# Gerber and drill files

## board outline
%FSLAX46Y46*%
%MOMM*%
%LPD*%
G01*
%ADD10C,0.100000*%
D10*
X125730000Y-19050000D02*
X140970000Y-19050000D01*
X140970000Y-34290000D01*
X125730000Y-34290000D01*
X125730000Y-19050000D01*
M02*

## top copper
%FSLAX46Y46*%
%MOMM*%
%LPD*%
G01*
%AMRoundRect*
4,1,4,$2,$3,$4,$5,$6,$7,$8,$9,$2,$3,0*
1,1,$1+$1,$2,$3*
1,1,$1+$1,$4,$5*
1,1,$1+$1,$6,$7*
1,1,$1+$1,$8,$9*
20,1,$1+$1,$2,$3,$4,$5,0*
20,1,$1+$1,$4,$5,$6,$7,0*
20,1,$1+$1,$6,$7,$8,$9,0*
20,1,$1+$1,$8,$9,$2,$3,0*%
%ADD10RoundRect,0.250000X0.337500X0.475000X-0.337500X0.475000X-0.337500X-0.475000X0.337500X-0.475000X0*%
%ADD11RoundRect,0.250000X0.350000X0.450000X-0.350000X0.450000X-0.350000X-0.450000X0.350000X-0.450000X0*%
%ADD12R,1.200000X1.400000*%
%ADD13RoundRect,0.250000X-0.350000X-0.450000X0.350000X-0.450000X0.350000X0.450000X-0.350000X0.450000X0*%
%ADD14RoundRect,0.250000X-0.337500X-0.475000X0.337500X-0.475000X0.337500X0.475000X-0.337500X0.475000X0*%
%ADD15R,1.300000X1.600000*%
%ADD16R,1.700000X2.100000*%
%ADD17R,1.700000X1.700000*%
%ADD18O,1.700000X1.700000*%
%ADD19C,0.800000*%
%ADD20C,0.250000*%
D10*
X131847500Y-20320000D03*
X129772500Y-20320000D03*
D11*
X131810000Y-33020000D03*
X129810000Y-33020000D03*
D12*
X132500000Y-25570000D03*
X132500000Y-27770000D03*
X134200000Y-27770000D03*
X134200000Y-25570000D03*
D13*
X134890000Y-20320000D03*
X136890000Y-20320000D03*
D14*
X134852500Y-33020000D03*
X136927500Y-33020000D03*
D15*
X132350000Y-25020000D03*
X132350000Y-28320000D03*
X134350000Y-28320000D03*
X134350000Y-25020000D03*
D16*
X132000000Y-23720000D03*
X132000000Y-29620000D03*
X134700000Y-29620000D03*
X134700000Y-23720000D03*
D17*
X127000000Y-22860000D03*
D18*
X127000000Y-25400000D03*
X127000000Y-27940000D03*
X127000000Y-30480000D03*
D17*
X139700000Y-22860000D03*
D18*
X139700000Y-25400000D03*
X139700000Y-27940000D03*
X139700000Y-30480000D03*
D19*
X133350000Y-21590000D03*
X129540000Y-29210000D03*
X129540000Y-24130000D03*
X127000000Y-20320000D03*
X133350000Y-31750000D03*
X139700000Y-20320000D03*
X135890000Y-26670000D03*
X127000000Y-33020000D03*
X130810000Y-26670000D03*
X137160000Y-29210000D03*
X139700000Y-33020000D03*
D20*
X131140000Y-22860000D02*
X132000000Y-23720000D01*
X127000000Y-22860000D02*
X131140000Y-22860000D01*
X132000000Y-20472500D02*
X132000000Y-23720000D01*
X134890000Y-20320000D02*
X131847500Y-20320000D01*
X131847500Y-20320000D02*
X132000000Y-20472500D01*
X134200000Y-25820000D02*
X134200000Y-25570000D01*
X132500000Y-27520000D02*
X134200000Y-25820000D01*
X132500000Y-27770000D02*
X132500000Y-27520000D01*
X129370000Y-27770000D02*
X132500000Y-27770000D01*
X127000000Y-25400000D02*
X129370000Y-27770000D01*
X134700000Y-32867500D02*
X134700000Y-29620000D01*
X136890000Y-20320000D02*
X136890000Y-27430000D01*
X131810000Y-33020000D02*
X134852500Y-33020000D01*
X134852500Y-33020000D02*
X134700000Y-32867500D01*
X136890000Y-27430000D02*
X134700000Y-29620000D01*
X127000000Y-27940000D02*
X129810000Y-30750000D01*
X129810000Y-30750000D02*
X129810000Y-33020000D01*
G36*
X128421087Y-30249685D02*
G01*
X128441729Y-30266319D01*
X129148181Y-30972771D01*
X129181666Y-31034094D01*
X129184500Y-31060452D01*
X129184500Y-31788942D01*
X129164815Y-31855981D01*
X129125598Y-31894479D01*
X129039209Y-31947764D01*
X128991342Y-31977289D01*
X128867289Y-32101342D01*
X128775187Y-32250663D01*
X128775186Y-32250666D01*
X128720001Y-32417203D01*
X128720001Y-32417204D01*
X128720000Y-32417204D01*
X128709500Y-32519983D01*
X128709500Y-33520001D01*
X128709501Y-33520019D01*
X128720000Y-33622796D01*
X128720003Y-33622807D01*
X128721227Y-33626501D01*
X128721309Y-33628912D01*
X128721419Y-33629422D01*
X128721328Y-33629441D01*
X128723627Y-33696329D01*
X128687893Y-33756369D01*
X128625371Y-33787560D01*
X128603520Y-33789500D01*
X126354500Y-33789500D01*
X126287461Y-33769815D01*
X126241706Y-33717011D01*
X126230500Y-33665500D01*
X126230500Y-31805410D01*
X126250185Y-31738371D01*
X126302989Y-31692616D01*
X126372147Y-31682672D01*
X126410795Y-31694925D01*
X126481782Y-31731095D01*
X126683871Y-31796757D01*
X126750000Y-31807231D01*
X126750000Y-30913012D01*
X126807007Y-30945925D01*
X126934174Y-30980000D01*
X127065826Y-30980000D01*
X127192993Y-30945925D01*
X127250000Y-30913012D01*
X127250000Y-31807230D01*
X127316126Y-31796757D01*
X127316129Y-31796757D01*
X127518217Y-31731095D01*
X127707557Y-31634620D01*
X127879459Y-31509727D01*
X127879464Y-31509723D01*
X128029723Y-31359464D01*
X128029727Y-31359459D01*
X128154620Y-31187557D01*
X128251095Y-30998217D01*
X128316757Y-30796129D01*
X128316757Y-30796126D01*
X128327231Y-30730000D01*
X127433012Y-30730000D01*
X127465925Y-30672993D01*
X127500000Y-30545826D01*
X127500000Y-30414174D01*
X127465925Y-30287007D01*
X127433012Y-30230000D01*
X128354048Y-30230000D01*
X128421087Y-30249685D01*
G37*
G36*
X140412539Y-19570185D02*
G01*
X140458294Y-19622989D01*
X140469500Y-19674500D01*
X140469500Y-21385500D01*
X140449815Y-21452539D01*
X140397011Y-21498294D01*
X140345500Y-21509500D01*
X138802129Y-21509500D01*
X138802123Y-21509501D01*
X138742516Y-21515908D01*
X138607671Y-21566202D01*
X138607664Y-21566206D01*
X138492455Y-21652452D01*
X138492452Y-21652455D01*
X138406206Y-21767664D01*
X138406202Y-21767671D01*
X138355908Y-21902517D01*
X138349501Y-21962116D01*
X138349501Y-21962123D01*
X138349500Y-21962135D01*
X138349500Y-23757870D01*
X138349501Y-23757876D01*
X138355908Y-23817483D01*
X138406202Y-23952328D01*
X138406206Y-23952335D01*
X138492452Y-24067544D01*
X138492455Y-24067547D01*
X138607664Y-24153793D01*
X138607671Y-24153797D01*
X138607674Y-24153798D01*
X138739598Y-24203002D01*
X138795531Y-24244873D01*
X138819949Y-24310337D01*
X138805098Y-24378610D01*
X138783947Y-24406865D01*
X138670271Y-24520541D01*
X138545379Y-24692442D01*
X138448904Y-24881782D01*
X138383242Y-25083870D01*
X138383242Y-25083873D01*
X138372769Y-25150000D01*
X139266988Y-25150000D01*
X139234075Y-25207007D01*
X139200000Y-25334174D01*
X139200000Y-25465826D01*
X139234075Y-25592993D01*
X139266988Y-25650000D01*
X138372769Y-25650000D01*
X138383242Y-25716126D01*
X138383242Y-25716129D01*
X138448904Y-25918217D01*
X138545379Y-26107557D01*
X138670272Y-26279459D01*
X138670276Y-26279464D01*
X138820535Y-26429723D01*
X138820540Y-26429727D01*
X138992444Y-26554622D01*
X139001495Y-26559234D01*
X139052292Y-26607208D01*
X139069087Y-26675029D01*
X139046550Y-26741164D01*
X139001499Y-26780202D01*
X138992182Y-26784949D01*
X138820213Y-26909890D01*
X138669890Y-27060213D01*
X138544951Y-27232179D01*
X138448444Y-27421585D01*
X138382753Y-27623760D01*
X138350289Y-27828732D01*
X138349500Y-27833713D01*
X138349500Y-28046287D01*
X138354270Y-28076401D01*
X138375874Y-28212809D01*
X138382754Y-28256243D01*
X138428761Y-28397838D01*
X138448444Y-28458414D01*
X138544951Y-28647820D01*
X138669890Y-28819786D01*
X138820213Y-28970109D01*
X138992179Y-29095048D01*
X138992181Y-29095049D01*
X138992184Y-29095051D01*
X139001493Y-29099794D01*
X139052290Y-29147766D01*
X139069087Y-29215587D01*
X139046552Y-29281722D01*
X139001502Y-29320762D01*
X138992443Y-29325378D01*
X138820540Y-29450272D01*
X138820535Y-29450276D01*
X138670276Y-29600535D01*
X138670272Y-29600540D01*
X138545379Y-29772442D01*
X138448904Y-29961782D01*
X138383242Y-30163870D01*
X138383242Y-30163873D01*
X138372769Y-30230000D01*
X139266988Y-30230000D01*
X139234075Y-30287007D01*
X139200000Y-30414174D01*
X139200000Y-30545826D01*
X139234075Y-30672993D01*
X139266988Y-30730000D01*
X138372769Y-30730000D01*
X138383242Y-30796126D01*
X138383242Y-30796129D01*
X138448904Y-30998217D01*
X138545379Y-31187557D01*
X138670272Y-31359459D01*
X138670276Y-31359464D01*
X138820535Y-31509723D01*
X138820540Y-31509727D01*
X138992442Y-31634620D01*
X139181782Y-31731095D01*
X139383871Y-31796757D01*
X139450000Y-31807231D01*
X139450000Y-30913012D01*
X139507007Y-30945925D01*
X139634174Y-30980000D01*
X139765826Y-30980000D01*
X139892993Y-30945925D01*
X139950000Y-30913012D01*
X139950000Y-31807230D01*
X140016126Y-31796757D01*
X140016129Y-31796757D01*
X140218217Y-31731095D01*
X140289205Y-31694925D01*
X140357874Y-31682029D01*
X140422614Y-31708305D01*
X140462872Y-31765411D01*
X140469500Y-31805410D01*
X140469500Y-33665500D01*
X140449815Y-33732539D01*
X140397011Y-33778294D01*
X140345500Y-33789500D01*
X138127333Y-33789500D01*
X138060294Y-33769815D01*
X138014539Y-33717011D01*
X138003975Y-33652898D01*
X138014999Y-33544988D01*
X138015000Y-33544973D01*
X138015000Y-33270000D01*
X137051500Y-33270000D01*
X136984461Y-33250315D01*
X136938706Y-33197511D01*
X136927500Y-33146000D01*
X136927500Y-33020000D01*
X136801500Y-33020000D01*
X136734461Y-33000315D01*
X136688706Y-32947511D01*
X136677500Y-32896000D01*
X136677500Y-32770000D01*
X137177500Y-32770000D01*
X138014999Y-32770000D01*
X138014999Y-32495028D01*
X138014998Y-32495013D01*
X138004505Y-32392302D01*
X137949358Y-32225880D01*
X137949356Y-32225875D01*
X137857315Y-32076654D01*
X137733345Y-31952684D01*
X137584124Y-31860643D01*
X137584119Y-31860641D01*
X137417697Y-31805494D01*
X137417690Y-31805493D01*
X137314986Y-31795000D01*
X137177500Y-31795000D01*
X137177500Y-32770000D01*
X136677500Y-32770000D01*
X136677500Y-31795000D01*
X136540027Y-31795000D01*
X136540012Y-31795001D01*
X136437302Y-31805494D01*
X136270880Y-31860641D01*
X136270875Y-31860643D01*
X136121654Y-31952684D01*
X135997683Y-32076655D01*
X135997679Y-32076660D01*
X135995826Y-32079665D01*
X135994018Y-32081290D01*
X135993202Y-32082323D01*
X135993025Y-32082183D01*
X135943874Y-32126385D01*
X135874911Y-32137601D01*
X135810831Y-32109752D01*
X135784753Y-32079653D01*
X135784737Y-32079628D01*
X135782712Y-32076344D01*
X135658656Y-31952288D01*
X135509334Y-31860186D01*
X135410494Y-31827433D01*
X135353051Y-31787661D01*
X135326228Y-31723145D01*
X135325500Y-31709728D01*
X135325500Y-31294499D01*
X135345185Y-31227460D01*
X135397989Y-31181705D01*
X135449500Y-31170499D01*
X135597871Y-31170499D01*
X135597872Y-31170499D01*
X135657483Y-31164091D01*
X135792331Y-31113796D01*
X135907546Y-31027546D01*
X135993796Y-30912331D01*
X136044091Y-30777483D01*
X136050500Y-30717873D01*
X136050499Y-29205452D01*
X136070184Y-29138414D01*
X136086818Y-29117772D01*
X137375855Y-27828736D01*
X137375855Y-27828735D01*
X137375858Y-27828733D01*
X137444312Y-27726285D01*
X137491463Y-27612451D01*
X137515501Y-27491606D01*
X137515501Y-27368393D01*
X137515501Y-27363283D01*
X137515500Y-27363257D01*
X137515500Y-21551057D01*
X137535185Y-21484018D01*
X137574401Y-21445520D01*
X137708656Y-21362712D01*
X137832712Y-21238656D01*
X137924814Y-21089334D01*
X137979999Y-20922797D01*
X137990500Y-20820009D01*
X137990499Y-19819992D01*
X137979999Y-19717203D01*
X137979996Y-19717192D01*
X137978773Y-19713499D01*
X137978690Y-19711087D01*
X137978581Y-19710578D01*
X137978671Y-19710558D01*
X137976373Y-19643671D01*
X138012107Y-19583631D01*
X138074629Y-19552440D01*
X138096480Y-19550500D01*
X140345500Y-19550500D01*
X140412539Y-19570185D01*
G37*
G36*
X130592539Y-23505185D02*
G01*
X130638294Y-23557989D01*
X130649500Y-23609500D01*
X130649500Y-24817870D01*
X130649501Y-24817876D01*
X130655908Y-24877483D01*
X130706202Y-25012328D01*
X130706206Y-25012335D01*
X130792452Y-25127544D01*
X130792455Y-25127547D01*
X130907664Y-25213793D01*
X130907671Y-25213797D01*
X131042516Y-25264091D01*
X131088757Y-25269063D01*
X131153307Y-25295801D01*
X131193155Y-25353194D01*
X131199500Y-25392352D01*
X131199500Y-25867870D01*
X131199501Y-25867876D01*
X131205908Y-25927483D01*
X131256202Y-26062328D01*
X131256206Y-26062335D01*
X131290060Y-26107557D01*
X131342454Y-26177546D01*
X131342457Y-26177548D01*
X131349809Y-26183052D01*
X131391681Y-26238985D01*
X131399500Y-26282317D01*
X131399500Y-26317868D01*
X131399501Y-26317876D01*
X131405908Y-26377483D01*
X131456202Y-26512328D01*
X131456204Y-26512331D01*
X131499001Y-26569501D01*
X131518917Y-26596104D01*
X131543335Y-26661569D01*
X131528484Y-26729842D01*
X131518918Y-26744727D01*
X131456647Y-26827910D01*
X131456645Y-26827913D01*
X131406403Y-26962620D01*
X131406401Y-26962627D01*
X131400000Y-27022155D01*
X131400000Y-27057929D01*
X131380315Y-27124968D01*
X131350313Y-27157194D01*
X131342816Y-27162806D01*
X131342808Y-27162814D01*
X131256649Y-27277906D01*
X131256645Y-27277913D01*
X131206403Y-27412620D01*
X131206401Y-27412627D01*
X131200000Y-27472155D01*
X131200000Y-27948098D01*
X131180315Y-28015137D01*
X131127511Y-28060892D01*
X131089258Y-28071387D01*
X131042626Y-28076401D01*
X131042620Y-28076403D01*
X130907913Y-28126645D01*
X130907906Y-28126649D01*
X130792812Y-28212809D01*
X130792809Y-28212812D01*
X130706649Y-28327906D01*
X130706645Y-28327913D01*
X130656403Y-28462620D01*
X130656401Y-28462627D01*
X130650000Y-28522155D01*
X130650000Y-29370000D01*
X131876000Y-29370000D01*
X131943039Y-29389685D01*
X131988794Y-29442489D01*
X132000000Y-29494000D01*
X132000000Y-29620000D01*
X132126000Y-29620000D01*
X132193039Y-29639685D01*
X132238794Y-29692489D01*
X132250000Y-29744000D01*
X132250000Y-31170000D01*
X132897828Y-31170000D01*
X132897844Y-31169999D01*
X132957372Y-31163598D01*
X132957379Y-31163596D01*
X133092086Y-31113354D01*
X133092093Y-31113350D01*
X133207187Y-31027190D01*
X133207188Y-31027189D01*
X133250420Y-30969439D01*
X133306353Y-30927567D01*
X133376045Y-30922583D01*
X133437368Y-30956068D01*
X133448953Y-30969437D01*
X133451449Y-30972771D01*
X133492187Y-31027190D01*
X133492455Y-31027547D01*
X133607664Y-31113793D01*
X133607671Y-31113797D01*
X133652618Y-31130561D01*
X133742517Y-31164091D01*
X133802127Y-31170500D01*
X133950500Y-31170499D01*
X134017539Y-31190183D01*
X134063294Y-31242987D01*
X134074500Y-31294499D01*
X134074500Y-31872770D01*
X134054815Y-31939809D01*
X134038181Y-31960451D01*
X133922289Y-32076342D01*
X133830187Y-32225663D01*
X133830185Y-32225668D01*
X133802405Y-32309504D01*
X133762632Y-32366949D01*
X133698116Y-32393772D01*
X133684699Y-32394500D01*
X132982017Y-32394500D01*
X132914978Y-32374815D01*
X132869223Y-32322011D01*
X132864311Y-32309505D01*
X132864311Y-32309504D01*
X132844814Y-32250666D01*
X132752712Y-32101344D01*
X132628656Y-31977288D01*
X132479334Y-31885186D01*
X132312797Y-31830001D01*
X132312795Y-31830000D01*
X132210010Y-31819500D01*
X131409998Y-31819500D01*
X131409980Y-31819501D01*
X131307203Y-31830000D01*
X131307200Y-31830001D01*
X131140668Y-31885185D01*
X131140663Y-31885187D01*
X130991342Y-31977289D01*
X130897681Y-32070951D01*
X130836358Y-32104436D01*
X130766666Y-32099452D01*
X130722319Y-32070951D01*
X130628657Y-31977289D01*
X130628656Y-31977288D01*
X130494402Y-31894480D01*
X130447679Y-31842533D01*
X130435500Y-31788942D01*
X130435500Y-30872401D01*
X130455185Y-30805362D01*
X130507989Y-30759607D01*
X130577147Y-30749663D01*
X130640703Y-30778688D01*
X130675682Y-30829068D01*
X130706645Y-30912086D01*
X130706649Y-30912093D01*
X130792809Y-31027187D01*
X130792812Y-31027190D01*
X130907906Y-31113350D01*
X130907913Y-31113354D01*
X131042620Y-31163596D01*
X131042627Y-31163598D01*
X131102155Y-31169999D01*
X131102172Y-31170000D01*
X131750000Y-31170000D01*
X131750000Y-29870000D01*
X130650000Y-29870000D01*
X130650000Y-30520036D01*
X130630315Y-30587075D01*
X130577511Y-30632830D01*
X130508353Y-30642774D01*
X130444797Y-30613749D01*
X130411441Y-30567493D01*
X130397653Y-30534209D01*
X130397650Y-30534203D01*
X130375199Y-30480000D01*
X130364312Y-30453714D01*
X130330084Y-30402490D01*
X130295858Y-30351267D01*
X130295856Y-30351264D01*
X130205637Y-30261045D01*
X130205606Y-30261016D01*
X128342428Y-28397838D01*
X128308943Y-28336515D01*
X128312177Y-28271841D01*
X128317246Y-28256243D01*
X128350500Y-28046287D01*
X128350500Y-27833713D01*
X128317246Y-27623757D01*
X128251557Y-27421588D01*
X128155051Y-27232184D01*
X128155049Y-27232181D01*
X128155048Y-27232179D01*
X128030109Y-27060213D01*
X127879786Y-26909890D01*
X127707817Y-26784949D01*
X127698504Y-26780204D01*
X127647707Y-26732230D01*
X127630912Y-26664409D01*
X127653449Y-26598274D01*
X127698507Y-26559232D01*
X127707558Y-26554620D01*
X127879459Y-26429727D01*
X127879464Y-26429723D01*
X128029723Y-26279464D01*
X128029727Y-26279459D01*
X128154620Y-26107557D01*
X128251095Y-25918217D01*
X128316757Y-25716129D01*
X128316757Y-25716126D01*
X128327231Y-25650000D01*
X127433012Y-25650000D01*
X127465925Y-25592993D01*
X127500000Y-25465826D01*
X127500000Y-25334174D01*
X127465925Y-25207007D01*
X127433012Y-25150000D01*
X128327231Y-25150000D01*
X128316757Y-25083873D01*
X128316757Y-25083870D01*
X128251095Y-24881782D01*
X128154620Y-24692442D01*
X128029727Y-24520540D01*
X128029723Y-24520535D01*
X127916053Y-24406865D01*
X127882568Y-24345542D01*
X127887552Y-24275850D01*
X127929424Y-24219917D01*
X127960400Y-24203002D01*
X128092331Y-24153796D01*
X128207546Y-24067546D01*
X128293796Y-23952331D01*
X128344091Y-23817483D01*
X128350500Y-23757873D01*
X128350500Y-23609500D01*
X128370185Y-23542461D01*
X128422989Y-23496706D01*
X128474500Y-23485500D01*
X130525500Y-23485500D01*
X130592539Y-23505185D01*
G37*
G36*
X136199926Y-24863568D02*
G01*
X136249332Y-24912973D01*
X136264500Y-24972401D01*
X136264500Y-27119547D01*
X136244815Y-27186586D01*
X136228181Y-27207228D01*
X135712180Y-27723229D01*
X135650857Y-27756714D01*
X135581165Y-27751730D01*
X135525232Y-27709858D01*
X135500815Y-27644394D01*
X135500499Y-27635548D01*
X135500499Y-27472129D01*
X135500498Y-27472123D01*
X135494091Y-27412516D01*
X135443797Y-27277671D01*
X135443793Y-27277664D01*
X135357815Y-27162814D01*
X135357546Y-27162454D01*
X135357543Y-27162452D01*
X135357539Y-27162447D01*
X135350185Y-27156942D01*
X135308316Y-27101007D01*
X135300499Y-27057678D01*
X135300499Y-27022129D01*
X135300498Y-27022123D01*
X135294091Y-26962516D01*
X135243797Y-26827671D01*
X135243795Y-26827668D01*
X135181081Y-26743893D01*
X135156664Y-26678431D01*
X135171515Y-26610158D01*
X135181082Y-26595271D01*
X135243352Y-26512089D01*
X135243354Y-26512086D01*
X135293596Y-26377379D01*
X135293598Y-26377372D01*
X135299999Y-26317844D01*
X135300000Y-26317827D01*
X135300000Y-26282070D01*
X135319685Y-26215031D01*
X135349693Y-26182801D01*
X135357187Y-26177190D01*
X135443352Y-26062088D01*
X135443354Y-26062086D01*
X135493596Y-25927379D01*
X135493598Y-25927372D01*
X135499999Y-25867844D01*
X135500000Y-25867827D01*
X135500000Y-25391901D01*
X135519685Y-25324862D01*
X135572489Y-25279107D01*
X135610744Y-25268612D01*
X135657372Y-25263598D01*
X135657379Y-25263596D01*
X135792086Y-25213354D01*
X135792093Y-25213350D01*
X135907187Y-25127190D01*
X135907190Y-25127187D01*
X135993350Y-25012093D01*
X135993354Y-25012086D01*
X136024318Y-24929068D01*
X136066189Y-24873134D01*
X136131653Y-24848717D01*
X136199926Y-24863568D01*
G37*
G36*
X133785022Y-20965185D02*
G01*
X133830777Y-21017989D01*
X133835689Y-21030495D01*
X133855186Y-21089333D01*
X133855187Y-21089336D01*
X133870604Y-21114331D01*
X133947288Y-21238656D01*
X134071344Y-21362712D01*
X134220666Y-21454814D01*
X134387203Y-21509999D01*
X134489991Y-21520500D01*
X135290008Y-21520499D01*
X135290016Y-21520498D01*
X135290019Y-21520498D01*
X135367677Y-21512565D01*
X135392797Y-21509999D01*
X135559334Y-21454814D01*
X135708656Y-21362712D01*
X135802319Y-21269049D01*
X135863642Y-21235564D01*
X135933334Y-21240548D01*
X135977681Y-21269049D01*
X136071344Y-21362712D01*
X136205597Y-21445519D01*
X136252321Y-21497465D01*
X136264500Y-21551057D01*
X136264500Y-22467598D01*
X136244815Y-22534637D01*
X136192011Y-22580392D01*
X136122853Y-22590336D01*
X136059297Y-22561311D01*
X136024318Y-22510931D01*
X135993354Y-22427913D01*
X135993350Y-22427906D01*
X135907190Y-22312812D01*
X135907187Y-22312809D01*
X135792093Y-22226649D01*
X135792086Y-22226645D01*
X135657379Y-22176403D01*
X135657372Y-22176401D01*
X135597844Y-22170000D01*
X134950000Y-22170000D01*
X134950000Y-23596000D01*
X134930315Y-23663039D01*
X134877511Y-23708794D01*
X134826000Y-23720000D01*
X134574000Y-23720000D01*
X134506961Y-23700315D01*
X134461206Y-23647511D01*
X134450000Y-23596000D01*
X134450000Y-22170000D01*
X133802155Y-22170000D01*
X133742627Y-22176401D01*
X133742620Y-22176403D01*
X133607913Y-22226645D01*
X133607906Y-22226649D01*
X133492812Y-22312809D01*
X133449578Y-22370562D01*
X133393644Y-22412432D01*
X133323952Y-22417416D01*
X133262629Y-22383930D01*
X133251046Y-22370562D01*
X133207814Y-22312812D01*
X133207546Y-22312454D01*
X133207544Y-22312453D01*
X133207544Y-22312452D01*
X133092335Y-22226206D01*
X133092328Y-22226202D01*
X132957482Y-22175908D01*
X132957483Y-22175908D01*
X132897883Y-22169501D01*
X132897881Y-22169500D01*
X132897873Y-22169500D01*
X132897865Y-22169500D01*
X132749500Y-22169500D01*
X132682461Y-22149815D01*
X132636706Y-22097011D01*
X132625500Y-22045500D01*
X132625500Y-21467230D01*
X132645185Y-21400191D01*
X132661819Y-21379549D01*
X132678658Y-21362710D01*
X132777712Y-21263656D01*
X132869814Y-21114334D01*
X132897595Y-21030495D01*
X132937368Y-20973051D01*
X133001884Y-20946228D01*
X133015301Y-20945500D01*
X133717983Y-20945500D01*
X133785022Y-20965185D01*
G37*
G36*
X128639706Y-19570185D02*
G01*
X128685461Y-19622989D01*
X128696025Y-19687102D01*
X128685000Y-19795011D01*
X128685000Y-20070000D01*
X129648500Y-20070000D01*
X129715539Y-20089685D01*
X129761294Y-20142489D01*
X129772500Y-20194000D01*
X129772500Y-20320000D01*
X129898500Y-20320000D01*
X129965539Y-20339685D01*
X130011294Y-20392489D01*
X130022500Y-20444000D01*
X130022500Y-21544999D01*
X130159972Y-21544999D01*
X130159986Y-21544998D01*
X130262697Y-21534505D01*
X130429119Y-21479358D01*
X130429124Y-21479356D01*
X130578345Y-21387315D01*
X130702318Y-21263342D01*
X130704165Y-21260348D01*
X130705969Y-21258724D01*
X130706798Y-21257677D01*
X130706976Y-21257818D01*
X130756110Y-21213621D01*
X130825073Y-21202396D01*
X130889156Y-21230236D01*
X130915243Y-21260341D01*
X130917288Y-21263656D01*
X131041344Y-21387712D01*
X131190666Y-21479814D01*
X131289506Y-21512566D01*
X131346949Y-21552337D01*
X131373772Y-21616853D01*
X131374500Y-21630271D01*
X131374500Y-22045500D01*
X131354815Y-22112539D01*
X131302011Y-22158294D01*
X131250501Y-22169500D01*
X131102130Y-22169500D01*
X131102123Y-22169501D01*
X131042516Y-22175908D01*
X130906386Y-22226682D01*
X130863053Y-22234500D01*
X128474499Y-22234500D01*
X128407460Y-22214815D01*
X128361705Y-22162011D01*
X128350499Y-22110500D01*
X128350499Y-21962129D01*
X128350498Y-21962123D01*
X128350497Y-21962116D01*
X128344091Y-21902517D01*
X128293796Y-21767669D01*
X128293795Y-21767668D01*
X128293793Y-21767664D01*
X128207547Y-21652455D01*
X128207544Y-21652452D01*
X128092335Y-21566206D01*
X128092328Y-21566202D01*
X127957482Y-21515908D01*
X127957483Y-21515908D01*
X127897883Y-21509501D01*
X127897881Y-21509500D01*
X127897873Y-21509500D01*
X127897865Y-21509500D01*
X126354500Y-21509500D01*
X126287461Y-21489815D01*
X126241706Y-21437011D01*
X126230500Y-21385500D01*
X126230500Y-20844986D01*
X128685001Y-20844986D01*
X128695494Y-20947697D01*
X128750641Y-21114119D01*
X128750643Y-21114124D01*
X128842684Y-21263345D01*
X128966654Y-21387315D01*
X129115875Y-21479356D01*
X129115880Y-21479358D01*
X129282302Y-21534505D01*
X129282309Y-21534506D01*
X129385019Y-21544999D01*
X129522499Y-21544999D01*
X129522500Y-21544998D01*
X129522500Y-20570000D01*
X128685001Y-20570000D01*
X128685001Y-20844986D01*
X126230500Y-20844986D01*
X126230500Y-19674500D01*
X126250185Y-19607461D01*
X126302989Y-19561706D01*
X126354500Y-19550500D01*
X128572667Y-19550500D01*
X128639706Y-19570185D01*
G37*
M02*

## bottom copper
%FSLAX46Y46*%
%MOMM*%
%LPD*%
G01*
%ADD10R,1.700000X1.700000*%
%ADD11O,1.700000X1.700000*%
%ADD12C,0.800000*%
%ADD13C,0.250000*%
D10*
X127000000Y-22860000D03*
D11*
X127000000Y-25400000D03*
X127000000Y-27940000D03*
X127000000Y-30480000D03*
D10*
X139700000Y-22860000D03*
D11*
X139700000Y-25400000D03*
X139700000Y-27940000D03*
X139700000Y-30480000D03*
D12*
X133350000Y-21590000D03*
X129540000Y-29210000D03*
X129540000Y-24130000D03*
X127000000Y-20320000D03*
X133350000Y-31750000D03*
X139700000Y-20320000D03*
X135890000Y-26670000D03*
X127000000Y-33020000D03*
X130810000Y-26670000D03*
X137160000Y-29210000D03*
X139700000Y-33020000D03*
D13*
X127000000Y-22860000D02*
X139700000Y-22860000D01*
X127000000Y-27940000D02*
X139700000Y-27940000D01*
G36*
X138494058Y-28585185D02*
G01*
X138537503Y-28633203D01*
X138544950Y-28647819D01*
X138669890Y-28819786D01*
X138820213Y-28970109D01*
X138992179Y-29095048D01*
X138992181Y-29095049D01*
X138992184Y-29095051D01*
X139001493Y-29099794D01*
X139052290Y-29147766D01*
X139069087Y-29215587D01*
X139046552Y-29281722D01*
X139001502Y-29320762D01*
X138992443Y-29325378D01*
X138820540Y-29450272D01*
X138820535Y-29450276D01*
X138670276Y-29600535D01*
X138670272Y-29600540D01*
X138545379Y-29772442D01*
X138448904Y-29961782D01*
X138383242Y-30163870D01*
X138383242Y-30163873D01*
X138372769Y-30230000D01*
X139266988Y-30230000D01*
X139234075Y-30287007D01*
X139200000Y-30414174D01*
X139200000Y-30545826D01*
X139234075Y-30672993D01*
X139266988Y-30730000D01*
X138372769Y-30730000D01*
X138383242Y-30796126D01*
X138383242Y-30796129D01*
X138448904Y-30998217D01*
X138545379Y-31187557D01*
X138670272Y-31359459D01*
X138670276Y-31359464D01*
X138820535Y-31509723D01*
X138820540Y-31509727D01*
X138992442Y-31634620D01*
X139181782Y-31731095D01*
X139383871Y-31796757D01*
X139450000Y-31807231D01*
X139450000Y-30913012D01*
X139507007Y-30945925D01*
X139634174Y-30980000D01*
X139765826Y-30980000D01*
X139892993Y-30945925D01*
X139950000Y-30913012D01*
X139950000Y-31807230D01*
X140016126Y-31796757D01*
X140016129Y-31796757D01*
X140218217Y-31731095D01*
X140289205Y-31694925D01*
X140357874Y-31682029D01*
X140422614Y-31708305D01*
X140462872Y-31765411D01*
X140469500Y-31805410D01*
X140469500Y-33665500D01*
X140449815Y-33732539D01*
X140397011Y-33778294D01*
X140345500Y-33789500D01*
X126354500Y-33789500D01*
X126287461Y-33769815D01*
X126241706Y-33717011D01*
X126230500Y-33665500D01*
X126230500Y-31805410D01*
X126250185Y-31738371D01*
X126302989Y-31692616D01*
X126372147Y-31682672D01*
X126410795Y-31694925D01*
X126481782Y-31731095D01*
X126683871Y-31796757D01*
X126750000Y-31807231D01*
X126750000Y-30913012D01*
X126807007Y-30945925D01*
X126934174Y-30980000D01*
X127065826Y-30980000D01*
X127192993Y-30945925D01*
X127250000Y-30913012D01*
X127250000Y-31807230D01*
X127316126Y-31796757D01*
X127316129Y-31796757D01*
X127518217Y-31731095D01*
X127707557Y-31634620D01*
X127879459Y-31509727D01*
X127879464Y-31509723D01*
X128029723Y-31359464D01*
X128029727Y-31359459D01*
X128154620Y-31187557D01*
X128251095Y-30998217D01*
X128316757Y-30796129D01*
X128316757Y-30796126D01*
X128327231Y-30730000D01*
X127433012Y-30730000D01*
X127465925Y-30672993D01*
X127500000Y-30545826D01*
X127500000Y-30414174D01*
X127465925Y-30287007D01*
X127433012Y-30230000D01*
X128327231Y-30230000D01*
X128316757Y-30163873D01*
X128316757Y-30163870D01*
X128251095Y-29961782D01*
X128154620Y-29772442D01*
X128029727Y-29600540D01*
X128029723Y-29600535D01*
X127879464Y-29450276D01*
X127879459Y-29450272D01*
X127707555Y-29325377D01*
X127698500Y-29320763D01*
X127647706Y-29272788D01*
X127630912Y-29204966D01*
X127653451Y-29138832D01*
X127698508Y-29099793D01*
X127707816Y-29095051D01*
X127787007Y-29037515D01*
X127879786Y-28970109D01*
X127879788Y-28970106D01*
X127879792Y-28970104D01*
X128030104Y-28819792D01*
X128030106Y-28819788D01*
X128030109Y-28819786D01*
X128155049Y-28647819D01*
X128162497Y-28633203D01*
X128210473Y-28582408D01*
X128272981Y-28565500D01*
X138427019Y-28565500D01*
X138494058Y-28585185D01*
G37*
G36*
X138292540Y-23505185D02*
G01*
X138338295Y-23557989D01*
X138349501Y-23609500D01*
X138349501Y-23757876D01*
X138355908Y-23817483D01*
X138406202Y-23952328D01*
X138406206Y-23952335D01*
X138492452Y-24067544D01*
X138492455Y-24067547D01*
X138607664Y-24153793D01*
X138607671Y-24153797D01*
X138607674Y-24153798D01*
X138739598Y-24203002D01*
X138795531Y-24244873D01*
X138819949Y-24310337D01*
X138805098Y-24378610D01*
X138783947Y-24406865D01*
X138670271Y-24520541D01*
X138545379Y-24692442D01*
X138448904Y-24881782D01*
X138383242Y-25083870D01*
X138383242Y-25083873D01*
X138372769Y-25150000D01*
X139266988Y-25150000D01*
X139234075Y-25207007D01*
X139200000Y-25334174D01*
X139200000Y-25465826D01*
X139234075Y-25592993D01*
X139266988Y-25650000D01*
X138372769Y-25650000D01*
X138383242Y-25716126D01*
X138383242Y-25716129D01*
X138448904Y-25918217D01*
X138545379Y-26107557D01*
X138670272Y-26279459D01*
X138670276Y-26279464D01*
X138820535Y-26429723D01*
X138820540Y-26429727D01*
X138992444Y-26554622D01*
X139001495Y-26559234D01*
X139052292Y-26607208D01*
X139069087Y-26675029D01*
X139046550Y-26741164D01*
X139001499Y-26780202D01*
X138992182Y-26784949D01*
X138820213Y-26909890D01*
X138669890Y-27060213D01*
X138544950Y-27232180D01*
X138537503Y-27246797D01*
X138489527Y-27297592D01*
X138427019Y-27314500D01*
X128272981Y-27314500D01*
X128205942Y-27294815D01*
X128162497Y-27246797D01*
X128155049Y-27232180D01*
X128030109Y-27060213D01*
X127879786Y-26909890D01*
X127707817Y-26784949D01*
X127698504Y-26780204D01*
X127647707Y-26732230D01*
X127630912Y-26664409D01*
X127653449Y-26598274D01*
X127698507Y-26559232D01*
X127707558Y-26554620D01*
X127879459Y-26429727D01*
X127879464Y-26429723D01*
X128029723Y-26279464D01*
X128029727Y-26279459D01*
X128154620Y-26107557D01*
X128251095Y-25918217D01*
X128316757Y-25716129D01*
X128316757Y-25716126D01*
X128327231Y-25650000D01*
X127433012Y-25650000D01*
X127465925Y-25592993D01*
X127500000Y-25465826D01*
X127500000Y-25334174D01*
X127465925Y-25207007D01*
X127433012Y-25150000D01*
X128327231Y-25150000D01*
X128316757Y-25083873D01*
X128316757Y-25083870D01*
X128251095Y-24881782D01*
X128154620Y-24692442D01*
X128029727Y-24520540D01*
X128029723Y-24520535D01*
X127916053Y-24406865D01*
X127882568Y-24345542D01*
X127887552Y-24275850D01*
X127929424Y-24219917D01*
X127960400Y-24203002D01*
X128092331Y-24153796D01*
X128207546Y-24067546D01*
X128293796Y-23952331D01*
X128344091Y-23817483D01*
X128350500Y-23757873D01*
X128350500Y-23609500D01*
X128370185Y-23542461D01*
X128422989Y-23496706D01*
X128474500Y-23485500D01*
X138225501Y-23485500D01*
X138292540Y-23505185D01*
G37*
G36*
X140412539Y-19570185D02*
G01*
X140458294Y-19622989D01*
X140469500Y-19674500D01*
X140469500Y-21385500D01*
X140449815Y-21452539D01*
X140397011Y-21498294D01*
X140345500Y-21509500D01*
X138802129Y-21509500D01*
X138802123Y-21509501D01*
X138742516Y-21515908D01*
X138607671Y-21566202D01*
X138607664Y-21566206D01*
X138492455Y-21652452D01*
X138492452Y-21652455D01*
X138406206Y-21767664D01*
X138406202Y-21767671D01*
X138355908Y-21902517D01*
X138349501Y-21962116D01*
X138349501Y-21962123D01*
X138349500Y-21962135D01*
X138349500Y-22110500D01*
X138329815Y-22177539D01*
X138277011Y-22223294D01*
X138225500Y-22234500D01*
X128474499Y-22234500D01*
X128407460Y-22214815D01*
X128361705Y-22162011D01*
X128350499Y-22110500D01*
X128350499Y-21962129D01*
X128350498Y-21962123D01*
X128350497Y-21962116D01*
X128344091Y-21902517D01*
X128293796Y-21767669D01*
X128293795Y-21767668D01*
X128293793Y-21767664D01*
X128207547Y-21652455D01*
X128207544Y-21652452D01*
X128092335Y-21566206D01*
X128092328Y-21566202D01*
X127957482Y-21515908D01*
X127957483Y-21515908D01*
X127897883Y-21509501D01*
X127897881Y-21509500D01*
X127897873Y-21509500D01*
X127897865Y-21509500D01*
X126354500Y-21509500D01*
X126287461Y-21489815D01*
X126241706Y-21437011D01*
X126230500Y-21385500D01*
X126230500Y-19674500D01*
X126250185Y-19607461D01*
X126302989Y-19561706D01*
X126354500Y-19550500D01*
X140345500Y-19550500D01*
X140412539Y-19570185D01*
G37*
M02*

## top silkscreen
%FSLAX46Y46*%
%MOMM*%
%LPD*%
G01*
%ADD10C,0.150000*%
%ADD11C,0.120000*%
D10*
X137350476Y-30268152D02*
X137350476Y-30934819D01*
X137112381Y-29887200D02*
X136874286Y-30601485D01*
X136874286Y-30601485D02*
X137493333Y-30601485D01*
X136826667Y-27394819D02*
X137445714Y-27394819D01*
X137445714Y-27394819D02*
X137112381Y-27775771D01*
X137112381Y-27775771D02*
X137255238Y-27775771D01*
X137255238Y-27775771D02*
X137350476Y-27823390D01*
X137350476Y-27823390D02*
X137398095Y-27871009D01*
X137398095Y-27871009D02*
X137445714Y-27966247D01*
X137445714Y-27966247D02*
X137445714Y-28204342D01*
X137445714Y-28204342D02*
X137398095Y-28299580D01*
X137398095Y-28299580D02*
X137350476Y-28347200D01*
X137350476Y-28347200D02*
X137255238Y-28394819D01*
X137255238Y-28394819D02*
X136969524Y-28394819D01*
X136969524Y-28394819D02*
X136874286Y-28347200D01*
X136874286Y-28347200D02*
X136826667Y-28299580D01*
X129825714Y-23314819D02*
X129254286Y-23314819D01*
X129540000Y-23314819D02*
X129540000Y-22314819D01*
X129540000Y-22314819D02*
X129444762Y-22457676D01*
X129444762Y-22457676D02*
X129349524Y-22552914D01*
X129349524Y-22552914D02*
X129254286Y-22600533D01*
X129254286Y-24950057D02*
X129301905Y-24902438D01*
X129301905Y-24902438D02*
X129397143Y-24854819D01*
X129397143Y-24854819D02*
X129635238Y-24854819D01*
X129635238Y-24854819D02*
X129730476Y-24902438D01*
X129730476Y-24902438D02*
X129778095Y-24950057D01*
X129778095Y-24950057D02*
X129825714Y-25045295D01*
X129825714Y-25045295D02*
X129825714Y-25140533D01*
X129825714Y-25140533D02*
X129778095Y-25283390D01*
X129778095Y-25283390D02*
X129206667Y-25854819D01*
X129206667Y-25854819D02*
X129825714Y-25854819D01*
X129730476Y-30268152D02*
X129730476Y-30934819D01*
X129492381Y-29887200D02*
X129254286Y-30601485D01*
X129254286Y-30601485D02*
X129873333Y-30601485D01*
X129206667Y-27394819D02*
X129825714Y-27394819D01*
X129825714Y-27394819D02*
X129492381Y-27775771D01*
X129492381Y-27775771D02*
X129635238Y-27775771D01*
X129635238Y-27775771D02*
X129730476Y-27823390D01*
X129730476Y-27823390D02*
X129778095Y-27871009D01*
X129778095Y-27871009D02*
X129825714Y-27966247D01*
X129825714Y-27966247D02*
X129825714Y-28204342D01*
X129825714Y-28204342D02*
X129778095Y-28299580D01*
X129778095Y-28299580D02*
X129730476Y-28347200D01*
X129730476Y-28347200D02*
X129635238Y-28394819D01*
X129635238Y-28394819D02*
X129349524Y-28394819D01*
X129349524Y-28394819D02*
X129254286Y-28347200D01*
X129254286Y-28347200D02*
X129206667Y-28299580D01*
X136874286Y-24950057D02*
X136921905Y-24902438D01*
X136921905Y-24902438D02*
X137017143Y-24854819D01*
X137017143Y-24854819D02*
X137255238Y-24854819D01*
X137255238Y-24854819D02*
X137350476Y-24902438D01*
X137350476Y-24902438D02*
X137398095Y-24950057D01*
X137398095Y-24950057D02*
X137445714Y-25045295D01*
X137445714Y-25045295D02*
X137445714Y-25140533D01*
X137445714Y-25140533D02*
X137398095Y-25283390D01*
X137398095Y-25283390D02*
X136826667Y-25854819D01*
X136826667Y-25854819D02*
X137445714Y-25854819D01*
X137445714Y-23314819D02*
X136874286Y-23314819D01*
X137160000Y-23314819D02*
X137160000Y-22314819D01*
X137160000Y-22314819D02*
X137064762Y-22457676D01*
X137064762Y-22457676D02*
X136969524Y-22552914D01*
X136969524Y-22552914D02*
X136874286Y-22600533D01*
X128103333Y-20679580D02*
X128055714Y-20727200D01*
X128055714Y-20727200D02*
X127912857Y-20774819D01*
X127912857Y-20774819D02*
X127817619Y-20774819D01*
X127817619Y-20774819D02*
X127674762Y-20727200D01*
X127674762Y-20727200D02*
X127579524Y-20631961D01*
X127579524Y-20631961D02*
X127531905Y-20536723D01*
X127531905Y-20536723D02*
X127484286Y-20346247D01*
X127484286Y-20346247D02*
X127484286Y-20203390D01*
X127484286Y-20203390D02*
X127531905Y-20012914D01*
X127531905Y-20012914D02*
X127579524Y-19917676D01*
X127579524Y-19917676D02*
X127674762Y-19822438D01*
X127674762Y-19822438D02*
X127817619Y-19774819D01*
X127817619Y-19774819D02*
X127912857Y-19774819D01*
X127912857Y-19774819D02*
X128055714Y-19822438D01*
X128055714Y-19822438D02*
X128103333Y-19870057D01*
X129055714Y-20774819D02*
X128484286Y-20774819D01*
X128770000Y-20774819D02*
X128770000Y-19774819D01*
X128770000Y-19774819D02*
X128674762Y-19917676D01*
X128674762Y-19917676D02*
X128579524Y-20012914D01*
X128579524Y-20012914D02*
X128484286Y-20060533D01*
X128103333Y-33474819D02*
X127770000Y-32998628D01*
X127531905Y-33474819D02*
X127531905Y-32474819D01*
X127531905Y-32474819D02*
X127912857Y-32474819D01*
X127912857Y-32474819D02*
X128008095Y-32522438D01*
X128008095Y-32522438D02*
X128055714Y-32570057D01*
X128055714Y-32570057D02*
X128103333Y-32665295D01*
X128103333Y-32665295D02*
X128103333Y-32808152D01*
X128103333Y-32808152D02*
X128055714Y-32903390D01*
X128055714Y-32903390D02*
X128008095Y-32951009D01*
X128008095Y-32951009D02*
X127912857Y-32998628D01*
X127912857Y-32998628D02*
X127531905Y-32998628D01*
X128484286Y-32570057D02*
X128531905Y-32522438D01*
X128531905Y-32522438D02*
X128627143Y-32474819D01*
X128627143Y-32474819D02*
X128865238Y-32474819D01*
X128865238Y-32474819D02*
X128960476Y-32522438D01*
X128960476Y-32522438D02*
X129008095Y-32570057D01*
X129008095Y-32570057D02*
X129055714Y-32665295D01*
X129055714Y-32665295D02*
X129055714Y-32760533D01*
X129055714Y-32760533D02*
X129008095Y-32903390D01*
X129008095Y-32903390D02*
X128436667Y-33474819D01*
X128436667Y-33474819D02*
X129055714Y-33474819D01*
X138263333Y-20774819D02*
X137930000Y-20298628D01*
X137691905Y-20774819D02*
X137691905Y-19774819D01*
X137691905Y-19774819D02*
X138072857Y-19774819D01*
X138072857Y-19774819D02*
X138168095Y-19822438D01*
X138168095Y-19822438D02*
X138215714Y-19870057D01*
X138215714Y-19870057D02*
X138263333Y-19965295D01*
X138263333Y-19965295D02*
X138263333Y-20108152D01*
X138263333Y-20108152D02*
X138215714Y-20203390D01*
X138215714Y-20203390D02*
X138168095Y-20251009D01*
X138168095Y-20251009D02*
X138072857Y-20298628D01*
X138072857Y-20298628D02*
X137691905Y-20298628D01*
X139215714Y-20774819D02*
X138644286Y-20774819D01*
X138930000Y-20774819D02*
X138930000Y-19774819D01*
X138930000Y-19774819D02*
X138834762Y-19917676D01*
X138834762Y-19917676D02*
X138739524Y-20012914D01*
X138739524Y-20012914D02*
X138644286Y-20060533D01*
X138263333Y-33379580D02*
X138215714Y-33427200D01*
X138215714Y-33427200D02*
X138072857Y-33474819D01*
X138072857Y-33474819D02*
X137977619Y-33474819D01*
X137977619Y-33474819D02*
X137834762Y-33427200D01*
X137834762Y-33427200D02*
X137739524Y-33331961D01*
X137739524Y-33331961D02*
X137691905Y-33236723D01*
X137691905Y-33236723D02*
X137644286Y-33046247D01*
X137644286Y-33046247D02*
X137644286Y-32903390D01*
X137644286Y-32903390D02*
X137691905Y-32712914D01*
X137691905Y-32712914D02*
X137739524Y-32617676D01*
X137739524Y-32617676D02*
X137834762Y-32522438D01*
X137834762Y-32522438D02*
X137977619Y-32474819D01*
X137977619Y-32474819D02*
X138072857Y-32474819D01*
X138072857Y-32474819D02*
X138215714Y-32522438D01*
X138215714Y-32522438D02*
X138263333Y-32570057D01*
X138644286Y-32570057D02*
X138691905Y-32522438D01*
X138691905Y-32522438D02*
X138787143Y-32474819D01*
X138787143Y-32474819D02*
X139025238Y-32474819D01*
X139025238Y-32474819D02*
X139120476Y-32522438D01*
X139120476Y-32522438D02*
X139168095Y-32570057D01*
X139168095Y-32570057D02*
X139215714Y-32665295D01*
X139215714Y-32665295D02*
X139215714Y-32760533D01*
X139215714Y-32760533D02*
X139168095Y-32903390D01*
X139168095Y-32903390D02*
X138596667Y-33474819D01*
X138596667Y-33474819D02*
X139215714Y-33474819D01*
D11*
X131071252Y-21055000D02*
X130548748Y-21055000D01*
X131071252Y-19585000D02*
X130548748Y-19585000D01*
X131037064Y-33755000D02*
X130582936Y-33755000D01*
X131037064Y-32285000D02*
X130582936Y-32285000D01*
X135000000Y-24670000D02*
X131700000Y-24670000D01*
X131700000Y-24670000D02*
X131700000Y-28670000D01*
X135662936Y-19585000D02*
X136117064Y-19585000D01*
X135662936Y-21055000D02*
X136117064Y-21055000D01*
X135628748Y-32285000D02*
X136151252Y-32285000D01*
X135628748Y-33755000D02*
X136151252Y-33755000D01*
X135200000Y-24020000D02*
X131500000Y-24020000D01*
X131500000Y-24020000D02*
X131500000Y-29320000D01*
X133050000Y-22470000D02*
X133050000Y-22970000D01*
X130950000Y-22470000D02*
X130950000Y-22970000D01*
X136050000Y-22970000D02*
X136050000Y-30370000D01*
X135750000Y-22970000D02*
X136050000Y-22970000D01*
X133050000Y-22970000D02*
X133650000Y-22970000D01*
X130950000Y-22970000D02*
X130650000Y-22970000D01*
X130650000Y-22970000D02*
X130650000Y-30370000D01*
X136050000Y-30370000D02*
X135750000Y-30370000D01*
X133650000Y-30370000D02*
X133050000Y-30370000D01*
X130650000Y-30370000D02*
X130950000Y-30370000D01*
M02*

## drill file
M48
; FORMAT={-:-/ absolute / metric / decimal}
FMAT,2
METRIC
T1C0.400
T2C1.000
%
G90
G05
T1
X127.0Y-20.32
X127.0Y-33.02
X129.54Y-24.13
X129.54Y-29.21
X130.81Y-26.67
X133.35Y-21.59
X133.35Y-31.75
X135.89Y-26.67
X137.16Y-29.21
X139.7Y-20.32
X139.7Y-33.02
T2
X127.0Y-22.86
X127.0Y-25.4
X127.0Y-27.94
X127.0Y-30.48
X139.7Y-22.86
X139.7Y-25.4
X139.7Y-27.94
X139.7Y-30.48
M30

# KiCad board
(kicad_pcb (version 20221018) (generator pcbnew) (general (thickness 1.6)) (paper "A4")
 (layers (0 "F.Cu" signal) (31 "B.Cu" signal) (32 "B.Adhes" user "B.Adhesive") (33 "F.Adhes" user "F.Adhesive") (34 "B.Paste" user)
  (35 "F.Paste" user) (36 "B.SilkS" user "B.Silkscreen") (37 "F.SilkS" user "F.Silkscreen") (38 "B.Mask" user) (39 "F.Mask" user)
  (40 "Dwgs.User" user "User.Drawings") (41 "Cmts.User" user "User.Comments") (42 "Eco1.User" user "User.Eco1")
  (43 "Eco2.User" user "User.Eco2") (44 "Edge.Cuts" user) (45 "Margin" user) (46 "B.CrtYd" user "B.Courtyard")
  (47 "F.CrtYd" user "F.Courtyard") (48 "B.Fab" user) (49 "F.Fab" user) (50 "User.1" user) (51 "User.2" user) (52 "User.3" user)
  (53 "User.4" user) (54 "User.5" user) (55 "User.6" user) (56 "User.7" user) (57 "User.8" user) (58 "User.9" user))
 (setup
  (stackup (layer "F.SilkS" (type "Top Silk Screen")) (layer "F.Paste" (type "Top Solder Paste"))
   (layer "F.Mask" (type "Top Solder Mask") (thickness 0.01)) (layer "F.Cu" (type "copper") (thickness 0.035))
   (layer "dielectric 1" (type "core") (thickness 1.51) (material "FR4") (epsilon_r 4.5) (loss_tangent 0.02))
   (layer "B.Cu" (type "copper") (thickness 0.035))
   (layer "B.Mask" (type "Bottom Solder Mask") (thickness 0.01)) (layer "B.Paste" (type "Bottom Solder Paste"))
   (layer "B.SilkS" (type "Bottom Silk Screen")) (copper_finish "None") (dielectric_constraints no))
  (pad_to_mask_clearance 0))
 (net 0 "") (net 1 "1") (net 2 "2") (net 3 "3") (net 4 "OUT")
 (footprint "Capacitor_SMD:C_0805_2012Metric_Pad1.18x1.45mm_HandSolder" (layer "F.Cu") (at 130.81 20.32 180)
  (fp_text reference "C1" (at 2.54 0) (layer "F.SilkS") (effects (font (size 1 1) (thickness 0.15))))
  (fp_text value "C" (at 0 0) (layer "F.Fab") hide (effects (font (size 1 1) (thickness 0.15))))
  (fp_line (start -0.261252 -0.735) (end 0.261252 -0.735) (stroke (width 0.12) (type solid)) (layer "F.SilkS"))
  (fp_line (start -0.261252 0.735) (end 0.261252 0.735) (stroke (width 0.12) (type solid)) (layer "F.SilkS"))
  (pad "1" smd roundrect (at -1.0375 0 180) (size 1.175 1.45) (layers "F.Cu" "F.Paste" "F.Mask") (roundrect_rratio 0.212766) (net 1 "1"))
  (pad "2" smd roundrect (at 1.0375 0 180) (size 1.175 1.45) (layers "F.Cu" "F.Paste" "F.Mask") (roundrect_rratio 0.212766) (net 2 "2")))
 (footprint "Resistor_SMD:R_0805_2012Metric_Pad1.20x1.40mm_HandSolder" (layer "F.Cu") (at 130.81 33.02 180)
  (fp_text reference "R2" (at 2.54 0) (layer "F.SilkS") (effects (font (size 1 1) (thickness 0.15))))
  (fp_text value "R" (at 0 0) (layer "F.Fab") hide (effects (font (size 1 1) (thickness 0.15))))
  (fp_line (start -0.227064 -0.735) (end 0.227064 -0.735) (stroke (width 0.12) (type solid)) (layer "F.SilkS"))
  (fp_line (start -0.227064 0.735) (end 0.227064 0.735) (stroke (width 0.12) (type solid)) (layer "F.SilkS"))
  (pad "1" smd roundrect (at -1 0 180) (size 1.2 1.4) (layers "F.Cu" "F.Paste" "F.Mask") (roundrect_rratio 0.208333) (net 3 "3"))
  (pad "2" smd roundrect (at 1 0 180) (size 1.2 1.4) (layers "F.Cu" "F.Paste" "F.Mask") (roundrect_rratio 0.208333) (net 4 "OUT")))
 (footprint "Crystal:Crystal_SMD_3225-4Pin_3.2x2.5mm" (layer "F.Cu") (at 133.35 26.67 -90)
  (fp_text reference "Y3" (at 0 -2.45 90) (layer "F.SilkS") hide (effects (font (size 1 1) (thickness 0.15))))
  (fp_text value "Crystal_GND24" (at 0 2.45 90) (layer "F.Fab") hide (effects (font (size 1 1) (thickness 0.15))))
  (fp_line (start -2 -1.65) (end -2 1.65) (stroke (width 0.12) (type solid)) (layer "F.SilkS"))
  (fp_line (start -2 1.65) (end 2 1.65) (stroke (width 0.12) (type solid)) (layer "F.SilkS"))
  (pad "1" smd rect (at -1.1 0.85 270) (size 1.4 1.2) (layers "F.Cu" "F.Paste" "F.Mask") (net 1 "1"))
  (pad "2" smd rect (at 1.1 0.85 270) (size 1.4 1.2) (layers "F.Cu" "F.Paste" "F.Mask") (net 2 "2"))
  (pad "3" smd rect (at 1.1 -0.85 270) (size 1.4 1.2) (layers "F.Cu" "F.Paste" "F.Mask") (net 3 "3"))
  (pad "4" smd rect (at -1.1 -0.85 270) (size 1.4 1.2) (layers "F.Cu" "F.Paste" "F.Mask") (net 2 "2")))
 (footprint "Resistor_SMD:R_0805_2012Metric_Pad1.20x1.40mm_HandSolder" (layer "F.Cu") (at 135.89 20.32)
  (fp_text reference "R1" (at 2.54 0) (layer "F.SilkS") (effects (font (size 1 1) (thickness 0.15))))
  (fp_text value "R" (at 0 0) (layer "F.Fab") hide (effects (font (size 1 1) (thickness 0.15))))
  (fp_line (start -0.227064 -0.735) (end 0.227064 -0.735) (stroke (width 0.12) (type solid)) (layer "F.SilkS"))
  (fp_line (start -0.227064 0.735) (end 0.227064 0.735) (stroke (width 0.12) (type solid)) (layer "F.SilkS"))
  (pad "1" smd roundrect (at -1 0) (size 1.2 1.4) (layers "F.Cu" "F.Paste" "F.Mask") (roundrect_rratio 0.208333) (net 1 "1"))
  (pad "2" smd roundrect (at 1 0) (size 1.2 1.4) (layers "F.Cu" "F.Paste" "F.Mask") (roundrect_rratio 0.208333) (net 3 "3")))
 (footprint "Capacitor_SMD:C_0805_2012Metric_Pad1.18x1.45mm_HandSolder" (layer "F.Cu") (at 135.89 33.02)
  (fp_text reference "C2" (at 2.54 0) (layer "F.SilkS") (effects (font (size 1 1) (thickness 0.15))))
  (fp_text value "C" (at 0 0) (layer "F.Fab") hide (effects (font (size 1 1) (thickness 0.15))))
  (fp_line (start -0.261252 -0.735) (end 0.261252 -0.735) (stroke (width 0.12) (type solid)) (layer "F.SilkS"))
  (fp_line (start -0.261252 0.735) (end 0.261252 0.735) (stroke (width 0.12) (type solid)) (layer "F.SilkS"))
  (pad "1" smd roundrect (at -1.0375 0) (size 1.175 1.45) (layers "F.Cu" "F.Paste" "F.Mask") (roundrect_rratio 0.212766) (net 3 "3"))
  (pad "2" smd roundrect (at 1.0375 0) (size 1.175 1.45) (layers "F.Cu" "F.Paste" "F.Mask") (roundrect_rratio 0.212766) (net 2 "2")))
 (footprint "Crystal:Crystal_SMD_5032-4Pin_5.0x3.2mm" (layer "F.Cu") (at 133.35 26.67 -90)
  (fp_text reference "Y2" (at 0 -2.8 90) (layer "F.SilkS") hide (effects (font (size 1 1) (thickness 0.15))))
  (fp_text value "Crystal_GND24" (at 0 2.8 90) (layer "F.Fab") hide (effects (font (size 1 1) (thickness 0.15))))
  (fp_line (start -2.65 -1.85) (end -2.65 1.85) (stroke (width 0.12) (type solid)) (layer "F.SilkS"))
  (fp_line (start -2.65 1.85) (end 2.65 1.85) (stroke (width 0.12) (type solid)) (layer "F.SilkS"))
  (pad "1" smd rect (at -1.65 1 270) (size 1.6 1.3) (layers "F.Cu" "F.Paste" "F.Mask") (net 1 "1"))
  (pad "2" smd rect (at 1.65 1 270) (size 1.6 1.3) (layers "F.Cu" "F.Paste" "F.Mask") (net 2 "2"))
  (pad "3" smd rect (at 1.65 -1 270) (size 1.6 1.3) (layers "F.Cu" "F.Paste" "F.Mask") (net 3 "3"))
  (pad "4" smd rect (at -1.65 -1 270) (size 1.6 1.3) (layers "F.Cu" "F.Paste" "F.Mask") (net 2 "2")))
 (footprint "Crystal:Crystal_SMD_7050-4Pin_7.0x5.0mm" (layer "F.Cu") (at 133.35 26.67 -90)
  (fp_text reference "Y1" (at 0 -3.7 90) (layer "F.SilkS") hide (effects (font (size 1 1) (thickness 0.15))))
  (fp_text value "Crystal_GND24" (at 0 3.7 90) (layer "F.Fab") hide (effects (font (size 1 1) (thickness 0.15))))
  (fp_line (start -4.2 0.3) (end -3.7 0.3) (stroke (width 0.12) (type solid)) (layer "F.SilkS"))
  (fp_line (start -4.2 2.4) (end -3.7 2.4) (stroke (width 0.12) (type solid)) (layer "F.SilkS"))
  (fp_line (start -3.7 -2.7) (end 3.7 -2.7) (stroke (width 0.12) (type solid)) (layer "F.SilkS"))
  (fp_line (start -3.7 -2.4) (end -3.7 -2.7) (stroke (width 0.12) (type solid)) (layer "F.SilkS"))
  (fp_line (start -3.7 0.3) (end -3.7 -0.3) (stroke (width 0.12) (type solid)) (layer "F.SilkS"))
  (fp_line (start -3.7 2.4) (end -3.7 2.7) (stroke (width 0.12) (type solid)) (layer "F.SilkS"))
  (fp_line (start -3.7 2.7) (end 3.7 2.7) (stroke (width 0.12) (type solid)) (layer "F.SilkS"))
  (fp_line (start 3.7 -2.7) (end 3.7 -2.4) (stroke (width 0.12) (type solid)) (layer "F.SilkS"))
  (fp_line (start 3.7 -0.3) (end 3.7 0.3) (stroke (width 0.12) (type solid)) (layer "F.SilkS"))
  (fp_line (start 3.7 2.7) (end 3.7 2.4) (stroke (width 0.12) (type solid)) (layer "F.SilkS"))
  (pad "1" smd rect (at -2.95 1.35 270) (size 2.1 1.7) (layers "F.Cu" "F.Paste" "F.Mask") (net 1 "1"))
  (pad "2" smd rect (at 2.95 1.35 270) (size 2.1 1.7) (layers "F.Cu" "F.Paste" "F.Mask") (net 2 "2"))
  (pad "3" smd rect (at 2.95 -1.35 270) (size 2.1 1.7) (layers "F.Cu" "F.Paste" "F.Mask") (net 3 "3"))
  (pad "4" smd rect (at -2.95 -1.35 270) (size 2.1 1.7) (layers "F.Cu" "F.Paste" "F.Mask") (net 2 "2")))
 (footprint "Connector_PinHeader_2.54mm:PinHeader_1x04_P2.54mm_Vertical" (layer "B.Cu") (at 127 22.86 180)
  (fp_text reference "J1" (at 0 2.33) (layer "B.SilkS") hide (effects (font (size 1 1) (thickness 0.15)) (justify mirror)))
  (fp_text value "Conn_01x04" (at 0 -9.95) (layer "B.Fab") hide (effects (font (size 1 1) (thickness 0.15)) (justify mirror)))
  (pad "1" thru_hole rect (at 0 0 180) (size 1.7 1.7) (drill 1) (layers "*.Cu" "*.Mask") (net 1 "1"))
  (pad "2" thru_hole oval (at 0 -2.54 180) (size 1.7 1.7) (drill 1) (layers "*.Cu" "*.Mask") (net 2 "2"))
  (pad "3" thru_hole oval (at 0 -5.08 180) (size 1.7 1.7) (drill 1) (layers "*.Cu" "*.Mask") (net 4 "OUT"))
  (pad "4" thru_hole oval (at 0 -7.62 180) (size 1.7 1.7) (drill 1) (layers "*.Cu" "*.Mask") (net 2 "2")))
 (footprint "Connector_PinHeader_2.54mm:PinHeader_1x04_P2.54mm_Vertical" (layer "B.Cu") (at 139.7 22.86 180)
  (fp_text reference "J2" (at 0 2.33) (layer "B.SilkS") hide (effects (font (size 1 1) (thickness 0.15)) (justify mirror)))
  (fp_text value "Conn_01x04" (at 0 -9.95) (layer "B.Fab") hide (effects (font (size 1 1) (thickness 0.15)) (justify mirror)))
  (pad "1" thru_hole rect (at 0 0 180) (size 1.7 1.7) (drill 1) (layers "*.Cu" "*.Mask") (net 1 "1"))
  (pad "2" thru_hole oval (at 0 -2.54 180) (size 1.7 1.7) (drill 1) (layers "*.Cu" "*.Mask") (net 2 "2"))
  (pad "3" thru_hole oval (at 0 -5.08 180) (size 1.7 1.7) (drill 1) (layers "*.Cu" "*.Mask") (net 4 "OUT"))
  (pad "4" thru_hole oval (at 0 -7.62 180) (size 1.7 1.7) (drill 1) (layers "*.Cu" "*.Mask") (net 2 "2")))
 (gr_rect (start 125.73 19.05) (end 140.97 34.29) (stroke (width 0.1) (type default)) (fill none) (layer "Edge.Cuts"))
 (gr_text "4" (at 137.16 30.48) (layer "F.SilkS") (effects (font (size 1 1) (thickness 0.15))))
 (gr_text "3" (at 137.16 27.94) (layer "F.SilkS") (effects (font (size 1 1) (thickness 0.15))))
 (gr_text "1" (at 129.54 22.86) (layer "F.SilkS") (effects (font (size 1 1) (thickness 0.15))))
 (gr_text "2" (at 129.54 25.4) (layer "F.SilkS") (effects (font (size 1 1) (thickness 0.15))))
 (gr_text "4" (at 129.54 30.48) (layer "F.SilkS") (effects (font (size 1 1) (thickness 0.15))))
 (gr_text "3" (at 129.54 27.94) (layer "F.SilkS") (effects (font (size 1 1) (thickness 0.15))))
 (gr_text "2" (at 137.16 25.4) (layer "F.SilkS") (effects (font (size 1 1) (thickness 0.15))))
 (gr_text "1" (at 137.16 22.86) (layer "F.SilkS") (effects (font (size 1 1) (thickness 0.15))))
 (segment (start 131.14 22.86) (end 132 23.72) (width 0.25) (layer "F.Cu") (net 1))
 (segment (start 127 22.86) (end 131.14 22.86) (width 0.25) (layer "F.Cu") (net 1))
 (segment (start 132 20.4725) (end 132 23.72) (width 0.25) (layer "F.Cu") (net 1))
 (segment (start 134.89 20.32) (end 131.8475 20.32) (width 0.25) (layer "F.Cu") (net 1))
 (segment (start 131.8475 20.32) (end 132 20.4725) (width 0.25) (layer "F.Cu") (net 1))
 (segment (start 127 22.86) (end 139.7 22.86) (width 0.25) (layer "B.Cu") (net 1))
 (segment (start 134.2 25.82) (end 134.2 25.57) (width 0.25) (layer "F.Cu") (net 2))
 (segment (start 132.5 27.52) (end 134.2 25.82) (width 0.25) (layer "F.Cu") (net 2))
 (segment (start 132.5 27.77) (end 132.5 27.52) (width 0.25) (layer "F.Cu") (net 2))
 (segment (start 129.37 27.77) (end 132.5 27.77) (width 0.25) (layer "F.Cu") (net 2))
 (segment (start 127 25.4) (end 129.37 27.77) (width 0.25) (layer "F.Cu") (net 2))
 (via (at 133.35 21.59) (size 0.8) (drill 0.4) (layers "F.Cu" "B.Cu") (free) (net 2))
 (via (at 129.54 29.21) (size 0.8) (drill 0.4) (layers "F.Cu" "B.Cu") (free) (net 2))
 (via (at 129.54 24.13) (size 0.8) (drill 0.4) (layers "F.Cu" "B.Cu") (free) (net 2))
 (via (at 127 20.32) (size 0.8) (drill 0.4) (layers "F.Cu" "B.Cu") (free) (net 2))
 (via (at 133.35 31.75) (size 0.8) (drill 0.4) (layers "F.Cu" "B.Cu") (free) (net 2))
 (via (at 139.7 20.32) (size 0.8) (drill 0.4) (layers "F.Cu" "B.Cu") (free) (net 2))
 (via (at 135.89 26.67) (size 0.8) (drill 0.4) (layers "F.Cu" "B.Cu") (free) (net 2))
 (via (at 127 33.02) (size 0.8) (drill 0.4) (layers "F.Cu" "B.Cu") (free) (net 2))
 (via (at 130.81 26.67) (size 0.8) (drill 0.4) (layers "F.Cu" "B.Cu") (free) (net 2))
 (via (at 137.16 29.21) (size 0.8) (drill 0.4) (layers "F.Cu" "B.Cu") (free) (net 2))
 (via (at 139.7 33.02) (size 0.8) (drill 0.4) (layers "F.Cu" "B.Cu") (free) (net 2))
 (segment (start 134.7 32.8675) (end 134.7 29.62) (width 0.25) (layer "F.Cu") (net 3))
 (segment (start 136.89 20.32) (end 136.89 27.43) (width 0.25) (layer "F.Cu") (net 3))
 (segment (start 131.81 33.02) (end 134.8525 33.02) (width 0.25) (layer "F.Cu") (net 3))
 (segment (start 134.8525 33.02) (end 134.7 32.8675) (width 0.25) (layer "F.Cu") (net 3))
 (segment (start 136.89 27.43) (end 134.7 29.62) (width 0.25) (layer "F.Cu") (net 3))
 (segment (start 127 27.94) (end 129.81 30.75) (width 0.25) (layer "F.Cu") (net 4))
 (segment (start 129.81 30.75) (end 129.81 33.02) (width 0.25) (layer "F.Cu") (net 4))
 (segment (start 127 27.94) (end 139.7 27.94) (width 0.25) (layer "B.Cu") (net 4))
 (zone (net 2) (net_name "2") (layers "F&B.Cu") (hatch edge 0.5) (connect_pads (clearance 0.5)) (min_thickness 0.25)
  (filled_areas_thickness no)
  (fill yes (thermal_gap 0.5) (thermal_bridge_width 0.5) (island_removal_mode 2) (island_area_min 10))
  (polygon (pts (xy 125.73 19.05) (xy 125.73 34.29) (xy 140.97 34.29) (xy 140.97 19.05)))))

